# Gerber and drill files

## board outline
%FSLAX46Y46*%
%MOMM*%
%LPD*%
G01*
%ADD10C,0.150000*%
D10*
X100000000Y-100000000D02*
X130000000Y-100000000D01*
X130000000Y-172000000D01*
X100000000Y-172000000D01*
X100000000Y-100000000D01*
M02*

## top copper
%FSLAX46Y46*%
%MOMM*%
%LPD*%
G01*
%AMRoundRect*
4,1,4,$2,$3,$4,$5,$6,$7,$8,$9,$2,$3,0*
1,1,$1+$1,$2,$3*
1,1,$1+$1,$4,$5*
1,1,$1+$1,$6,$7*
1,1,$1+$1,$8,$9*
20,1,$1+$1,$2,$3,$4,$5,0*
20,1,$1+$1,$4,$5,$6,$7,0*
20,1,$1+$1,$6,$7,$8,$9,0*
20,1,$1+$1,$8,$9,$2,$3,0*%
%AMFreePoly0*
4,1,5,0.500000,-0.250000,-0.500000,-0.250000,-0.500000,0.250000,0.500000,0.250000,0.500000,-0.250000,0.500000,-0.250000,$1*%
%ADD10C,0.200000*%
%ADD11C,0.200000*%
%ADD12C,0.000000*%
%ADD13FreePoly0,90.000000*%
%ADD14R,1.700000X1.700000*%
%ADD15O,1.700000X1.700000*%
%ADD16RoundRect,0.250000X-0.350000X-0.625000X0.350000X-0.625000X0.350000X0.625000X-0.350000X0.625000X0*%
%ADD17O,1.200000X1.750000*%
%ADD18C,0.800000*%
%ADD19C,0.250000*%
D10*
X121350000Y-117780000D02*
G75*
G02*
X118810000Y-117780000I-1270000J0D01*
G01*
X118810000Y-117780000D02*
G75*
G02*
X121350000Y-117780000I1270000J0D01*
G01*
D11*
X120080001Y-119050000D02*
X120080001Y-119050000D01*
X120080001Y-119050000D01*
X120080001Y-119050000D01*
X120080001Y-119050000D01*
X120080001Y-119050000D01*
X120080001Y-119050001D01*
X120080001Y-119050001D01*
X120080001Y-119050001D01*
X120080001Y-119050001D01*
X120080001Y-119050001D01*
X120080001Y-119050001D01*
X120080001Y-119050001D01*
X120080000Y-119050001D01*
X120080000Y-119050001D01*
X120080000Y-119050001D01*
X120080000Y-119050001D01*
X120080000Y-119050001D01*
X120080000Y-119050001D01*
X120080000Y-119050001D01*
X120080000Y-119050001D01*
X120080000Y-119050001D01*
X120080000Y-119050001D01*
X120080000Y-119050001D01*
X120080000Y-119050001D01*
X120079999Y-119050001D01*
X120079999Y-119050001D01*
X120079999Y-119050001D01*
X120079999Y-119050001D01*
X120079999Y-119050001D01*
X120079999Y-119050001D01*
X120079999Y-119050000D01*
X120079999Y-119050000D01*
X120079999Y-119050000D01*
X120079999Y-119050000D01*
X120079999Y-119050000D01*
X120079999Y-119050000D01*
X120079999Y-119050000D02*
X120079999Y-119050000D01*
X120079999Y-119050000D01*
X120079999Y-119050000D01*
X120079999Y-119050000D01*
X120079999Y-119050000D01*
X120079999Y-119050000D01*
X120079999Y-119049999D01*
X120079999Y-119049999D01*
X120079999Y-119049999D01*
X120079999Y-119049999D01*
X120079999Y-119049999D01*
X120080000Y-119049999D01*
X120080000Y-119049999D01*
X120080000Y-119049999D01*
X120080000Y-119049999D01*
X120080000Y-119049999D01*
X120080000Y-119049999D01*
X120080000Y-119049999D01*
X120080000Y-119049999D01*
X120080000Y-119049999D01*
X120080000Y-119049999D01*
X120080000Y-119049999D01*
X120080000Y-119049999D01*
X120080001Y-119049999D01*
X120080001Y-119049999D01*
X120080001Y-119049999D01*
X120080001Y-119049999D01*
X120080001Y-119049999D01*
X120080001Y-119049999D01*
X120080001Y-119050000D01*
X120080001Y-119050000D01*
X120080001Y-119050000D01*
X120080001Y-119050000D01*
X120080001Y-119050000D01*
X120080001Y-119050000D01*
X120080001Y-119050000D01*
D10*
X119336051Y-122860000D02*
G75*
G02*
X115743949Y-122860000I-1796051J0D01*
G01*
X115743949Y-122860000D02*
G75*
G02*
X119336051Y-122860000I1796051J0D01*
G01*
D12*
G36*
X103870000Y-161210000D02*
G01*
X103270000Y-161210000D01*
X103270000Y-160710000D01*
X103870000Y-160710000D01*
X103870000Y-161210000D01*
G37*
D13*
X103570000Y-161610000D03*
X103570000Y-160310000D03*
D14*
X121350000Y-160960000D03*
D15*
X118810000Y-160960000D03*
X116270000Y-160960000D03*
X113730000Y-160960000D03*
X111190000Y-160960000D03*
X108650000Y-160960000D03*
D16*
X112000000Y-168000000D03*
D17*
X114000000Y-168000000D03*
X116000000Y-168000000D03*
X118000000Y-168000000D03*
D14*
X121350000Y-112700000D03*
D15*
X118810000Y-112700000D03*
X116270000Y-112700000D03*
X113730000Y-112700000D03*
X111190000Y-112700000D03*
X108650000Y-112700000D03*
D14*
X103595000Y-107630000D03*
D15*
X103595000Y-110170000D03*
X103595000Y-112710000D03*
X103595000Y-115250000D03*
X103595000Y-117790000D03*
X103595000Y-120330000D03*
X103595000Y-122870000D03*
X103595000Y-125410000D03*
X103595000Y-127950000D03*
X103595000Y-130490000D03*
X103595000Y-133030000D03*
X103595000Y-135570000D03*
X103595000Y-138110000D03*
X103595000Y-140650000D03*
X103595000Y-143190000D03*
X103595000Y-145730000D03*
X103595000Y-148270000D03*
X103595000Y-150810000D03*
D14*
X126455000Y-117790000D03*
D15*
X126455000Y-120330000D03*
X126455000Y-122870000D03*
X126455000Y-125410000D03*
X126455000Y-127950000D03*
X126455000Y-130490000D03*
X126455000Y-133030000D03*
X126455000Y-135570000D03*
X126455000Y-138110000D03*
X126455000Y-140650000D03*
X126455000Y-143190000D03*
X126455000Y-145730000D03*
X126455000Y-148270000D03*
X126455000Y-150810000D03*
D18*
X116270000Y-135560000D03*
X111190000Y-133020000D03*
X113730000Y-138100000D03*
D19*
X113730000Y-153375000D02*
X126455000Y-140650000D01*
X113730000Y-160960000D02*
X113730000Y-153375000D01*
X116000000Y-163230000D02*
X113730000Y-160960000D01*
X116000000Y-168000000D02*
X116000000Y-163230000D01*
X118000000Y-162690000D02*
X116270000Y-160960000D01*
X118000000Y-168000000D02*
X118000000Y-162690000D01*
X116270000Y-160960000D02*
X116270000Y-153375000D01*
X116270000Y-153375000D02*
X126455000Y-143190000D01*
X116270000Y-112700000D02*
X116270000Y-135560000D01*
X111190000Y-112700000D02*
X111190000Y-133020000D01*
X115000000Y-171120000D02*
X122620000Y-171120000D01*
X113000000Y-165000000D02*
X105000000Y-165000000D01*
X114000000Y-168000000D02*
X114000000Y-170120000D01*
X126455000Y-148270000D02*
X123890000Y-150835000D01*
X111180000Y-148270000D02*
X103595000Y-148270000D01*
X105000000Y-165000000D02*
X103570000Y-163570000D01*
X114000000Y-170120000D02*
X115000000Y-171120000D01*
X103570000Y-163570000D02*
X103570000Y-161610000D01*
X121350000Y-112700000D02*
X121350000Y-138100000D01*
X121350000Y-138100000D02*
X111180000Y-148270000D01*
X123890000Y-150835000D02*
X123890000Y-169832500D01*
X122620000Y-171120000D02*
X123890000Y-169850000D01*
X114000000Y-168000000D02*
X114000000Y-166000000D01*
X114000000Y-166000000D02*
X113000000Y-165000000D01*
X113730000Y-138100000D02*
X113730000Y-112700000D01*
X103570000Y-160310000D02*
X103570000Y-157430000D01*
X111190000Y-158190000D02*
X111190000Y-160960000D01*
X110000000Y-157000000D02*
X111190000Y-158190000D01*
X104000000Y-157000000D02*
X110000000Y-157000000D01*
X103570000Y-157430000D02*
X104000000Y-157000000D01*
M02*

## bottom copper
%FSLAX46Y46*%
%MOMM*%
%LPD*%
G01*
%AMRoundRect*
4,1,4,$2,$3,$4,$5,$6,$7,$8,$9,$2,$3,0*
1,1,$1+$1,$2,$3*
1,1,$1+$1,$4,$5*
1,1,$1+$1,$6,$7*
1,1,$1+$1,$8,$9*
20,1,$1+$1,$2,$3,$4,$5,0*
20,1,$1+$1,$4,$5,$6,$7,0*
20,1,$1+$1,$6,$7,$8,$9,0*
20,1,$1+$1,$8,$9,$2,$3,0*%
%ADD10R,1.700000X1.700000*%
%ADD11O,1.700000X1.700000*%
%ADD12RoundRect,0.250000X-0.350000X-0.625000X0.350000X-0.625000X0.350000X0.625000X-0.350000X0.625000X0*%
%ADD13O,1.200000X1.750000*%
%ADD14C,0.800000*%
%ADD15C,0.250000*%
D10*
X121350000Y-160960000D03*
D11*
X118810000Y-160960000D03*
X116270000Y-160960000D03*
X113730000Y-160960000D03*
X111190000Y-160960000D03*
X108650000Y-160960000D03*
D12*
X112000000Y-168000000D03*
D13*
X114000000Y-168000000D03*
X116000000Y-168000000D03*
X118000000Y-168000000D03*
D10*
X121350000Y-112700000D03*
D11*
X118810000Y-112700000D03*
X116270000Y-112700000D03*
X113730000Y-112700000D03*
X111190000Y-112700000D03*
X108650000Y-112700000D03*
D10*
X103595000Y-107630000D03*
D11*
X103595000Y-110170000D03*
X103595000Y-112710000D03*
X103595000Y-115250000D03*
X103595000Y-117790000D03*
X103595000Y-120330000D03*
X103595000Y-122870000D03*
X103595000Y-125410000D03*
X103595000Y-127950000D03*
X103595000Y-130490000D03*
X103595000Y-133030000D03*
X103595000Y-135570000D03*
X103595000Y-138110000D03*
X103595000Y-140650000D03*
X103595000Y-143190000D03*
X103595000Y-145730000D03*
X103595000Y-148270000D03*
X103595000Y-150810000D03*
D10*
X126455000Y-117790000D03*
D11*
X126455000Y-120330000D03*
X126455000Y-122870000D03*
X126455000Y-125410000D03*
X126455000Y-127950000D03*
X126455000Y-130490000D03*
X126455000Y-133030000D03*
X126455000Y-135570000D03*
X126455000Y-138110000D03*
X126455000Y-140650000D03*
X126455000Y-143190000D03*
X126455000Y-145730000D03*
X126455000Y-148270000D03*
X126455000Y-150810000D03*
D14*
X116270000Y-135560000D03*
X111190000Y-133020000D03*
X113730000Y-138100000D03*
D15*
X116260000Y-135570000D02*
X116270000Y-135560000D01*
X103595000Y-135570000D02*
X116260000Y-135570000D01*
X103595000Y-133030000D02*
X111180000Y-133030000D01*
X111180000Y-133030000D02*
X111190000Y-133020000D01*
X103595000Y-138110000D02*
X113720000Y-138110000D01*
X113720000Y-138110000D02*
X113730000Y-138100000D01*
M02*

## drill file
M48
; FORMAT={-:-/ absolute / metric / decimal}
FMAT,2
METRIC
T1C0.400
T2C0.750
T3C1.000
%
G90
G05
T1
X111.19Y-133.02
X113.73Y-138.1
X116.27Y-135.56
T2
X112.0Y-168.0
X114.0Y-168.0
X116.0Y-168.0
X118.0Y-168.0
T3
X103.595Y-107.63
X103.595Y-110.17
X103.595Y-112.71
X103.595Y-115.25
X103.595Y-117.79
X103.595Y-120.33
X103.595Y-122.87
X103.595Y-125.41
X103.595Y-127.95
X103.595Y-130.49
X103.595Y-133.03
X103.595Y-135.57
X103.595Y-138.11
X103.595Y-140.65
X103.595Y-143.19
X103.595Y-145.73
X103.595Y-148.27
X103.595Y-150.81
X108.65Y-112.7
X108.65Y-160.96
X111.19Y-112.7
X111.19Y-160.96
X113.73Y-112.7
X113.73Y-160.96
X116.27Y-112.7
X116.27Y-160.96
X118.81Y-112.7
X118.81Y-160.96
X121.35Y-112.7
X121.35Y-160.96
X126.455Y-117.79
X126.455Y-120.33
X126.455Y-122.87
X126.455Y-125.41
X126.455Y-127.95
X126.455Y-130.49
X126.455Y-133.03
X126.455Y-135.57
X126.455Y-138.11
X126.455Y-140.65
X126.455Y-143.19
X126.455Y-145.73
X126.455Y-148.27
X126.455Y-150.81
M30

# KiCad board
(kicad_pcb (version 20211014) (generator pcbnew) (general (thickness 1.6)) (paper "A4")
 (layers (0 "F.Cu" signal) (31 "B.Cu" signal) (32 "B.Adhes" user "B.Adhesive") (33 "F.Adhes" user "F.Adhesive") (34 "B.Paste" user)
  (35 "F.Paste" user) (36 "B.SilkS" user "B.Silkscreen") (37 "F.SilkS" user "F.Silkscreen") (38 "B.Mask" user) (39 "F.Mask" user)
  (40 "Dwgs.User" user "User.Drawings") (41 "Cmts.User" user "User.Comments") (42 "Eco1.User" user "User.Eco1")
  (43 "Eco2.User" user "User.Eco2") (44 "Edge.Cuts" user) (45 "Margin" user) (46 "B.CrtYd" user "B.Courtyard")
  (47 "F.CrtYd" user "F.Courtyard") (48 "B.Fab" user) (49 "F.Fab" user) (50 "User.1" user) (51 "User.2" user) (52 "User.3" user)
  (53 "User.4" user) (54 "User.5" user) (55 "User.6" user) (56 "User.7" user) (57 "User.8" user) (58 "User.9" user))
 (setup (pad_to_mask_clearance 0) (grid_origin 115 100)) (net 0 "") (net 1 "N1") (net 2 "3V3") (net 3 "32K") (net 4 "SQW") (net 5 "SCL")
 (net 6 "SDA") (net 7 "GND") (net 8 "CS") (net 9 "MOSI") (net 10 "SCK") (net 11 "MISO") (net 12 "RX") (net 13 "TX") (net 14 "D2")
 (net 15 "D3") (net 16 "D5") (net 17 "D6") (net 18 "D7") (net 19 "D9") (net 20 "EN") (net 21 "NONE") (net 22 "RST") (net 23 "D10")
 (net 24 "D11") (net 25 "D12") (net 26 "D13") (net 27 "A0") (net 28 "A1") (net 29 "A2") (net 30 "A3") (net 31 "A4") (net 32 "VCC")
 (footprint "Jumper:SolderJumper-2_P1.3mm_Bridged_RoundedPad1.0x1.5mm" (layer "F.Cu") (at 103.57 160.96 90)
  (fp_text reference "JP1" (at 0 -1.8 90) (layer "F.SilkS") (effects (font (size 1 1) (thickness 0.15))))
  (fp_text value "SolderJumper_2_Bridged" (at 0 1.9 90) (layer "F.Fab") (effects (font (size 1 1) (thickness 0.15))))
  (fp_poly (pts (xy 0.25 -0.3) (xy -0.25 -0.3) (xy -0.25 0.3) (xy 0.25 0.3)) (layer "F.Cu") (width 0) (fill solid))
  (pad "1" smd custom (at -0.65 0 90) (size 1 0.5) (layers "F.Cu" "F.Mask") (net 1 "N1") (zone_connect 2)
   (options (clearance outline) (anchor rect)) (primitives))
  (pad "2" smd custom (at 0.65 0 90) (size 1 0.5) (layers "F.Cu" "F.Mask") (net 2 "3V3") (zone_connect 2)
   (options (clearance outline) (anchor rect)) (primitives)))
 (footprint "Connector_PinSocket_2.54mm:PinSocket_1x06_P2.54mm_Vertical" (layer "F.Cu") (at 121.35 160.96 -90)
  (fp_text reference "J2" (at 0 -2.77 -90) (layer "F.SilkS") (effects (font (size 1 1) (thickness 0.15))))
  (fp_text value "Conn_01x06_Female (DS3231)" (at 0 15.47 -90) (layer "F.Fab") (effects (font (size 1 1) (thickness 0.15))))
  (pad "1" thru_hole rect (at 0 0 270) (size 1.7 1.7) (drill 1) (layers *.Cu *.Mask) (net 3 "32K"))
  (pad "2" thru_hole oval (at 0 2.54 270) (size 1.7 1.7) (drill 1) (layers *.Cu *.Mask) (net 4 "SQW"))
  (pad "3" thru_hole oval (at 0 5.08 270) (size 1.7 1.7) (drill 1) (layers *.Cu *.Mask) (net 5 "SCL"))
  (pad "4" thru_hole oval (at 0 7.62 270) (size 1.7 1.7) (drill 1) (layers *.Cu *.Mask) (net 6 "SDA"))
  (pad "5" thru_hole oval (at 0 10.16 270) (size 1.7 1.7) (drill 1) (layers *.Cu *.Mask) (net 1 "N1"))
  (pad "6" thru_hole oval (at 0 12.7 270) (size 1.7 1.7) (drill 1) (layers *.Cu *.Mask) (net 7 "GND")))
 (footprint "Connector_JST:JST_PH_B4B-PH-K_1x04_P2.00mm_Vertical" (layer "F.Cu") (at 112 168)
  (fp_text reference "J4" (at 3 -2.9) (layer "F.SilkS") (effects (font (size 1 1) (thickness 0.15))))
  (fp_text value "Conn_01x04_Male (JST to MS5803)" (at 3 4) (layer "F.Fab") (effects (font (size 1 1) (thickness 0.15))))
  (pad "1" thru_hole roundrect (at 0 0) (size 1.2 1.75) (drill 0.75) (layers *.Cu *.Mask) (roundrect_rratio 0.208333) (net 7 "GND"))
  (pad "2" thru_hole oval (at 2 0) (size 1.2 1.75) (drill 0.75) (layers *.Cu *.Mask) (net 2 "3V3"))
  (pad "3" thru_hole oval (at 4 0) (size 1.2 1.75) (drill 0.75) (layers *.Cu *.Mask) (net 6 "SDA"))
  (pad "4" thru_hole oval (at 6 0) (size 1.2 1.75) (drill 0.75) (layers *.Cu *.Mask) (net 5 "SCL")))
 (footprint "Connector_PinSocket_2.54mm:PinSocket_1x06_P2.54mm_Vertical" (layer "F.Cu") (at 121.35 112.7 -90)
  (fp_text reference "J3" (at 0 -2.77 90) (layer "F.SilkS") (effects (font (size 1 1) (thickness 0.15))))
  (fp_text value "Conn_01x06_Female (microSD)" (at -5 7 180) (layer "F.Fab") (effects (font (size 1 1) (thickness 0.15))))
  (pad "1" thru_hole rect (at 0 0 270) (size 1.7 1.7) (drill 1) (layers *.Cu *.Mask) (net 2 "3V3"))
  (pad "2" thru_hole oval (at 0 2.54 270) (size 1.7 1.7) (drill 1) (layers *.Cu *.Mask) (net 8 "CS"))
  (pad "3" thru_hole oval (at 0 5.08 270) (size 1.7 1.7) (drill 1) (layers *.Cu *.Mask) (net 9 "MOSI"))
  (pad "4" thru_hole oval (at 0 7.62 270) (size 1.7 1.7) (drill 1) (layers *.Cu *.Mask) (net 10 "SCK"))
  (pad "5" thru_hole oval (at 0 10.16 270) (size 1.7 1.7) (drill 1) (layers *.Cu *.Mask) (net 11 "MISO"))
  (pad "6" thru_hole oval (at 0 12.7 270) (size 1.7 1.7) (drill 1) (layers *.Cu *.Mask) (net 7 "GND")))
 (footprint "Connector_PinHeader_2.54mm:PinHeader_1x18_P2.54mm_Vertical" (layer "B.Cu") (at 103.595 107.63 180)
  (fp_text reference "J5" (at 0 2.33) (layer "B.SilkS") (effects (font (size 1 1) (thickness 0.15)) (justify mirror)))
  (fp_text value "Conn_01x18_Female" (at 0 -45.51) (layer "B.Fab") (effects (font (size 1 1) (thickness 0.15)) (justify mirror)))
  (pad "1" thru_hole rect (at 0 0 180) (size 1.7 1.7) (drill 1) (layers *.Cu *.Mask) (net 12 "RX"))
  (pad "2" thru_hole oval (at 0 -2.54 180) (size 1.7 1.7) (drill 1) (layers *.Cu *.Mask) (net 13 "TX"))
  (pad "3" thru_hole oval (at 0 -5.08 180) (size 1.7 1.7) (drill 1) (layers *.Cu *.Mask) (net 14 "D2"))
  (pad "4" thru_hole oval (at 0 -7.62 180) (size 1.7 1.7) (drill 1) (layers *.Cu *.Mask) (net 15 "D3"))
  (pad "5" thru_hole oval (at 0 -10.16 180) (size 1.7 1.7) (drill 1) (layers *.Cu *.Mask) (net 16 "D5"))
  (pad "6" thru_hole oval (at 0 -12.7 180) (size 1.7 1.7) (drill 1) (layers *.Cu *.Mask) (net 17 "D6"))
  (pad "7" thru_hole oval (at 0 -15.24 180) (size 1.7 1.7) (drill 1) (layers *.Cu *.Mask) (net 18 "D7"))
  (pad "8" thru_hole oval (at 0 -17.78 180) (size 1.7 1.7) (drill 1) (layers *.Cu *.Mask) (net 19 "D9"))
  (pad "9" thru_hole oval (at 0 -20.32 180) (size 1.7 1.7) (drill 1) (layers *.Cu *.Mask) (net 6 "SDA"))
  (pad "10" thru_hole oval (at 0 -22.86 180) (size 1.7 1.7) (drill 1) (layers *.Cu *.Mask) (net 5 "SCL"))
  (pad "11" thru_hole oval (at 0 -25.4 180) (size 1.7 1.7) (drill 1) (layers *.Cu *.Mask) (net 11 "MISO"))
  (pad "12" thru_hole oval (at 0 -27.94 180) (size 1.7 1.7) (drill 1) (layers *.Cu *.Mask) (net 9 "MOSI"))
  (pad "13" thru_hole oval (at 0 -30.48 180) (size 1.7 1.7) (drill 1) (layers *.Cu *.Mask) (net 10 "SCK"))
  (pad "14" thru_hole oval (at 0 -33.02 180) (size 1.7 1.7) (drill 1) (layers *.Cu *.Mask) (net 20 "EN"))
  (pad "15" thru_hole oval (at 0 -35.56 180) (size 1.7 1.7) (drill 1) (layers *.Cu *.Mask) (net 7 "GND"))
  (pad "16" thru_hole oval (at 0 -38.1 180) (size 1.7 1.7) (drill 1) (layers *.Cu *.Mask) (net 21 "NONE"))
  (pad "17" thru_hole oval (at 0 -40.64 180) (size 1.7 1.7) (drill 1) (layers *.Cu *.Mask) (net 2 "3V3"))
  (pad "18" thru_hole oval (at 0 -43.18 180) (size 1.7 1.7) (drill 1) (layers *.Cu *.Mask) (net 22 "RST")))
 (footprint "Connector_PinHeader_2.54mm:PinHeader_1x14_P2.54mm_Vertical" (layer "B.Cu") (at 126.455 117.79 180)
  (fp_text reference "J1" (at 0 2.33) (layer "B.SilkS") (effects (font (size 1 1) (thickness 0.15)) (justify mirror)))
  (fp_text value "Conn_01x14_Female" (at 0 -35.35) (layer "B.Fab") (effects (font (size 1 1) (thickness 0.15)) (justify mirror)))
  (pad "1" thru_hole rect (at 0 0 180) (size 1.7 1.7) (drill 1) (layers *.Cu *.Mask) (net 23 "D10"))
  (pad "2" thru_hole oval (at 0 -2.54 180) (size 1.7 1.7) (drill 1) (layers *.Cu *.Mask) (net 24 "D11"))
  (pad "3" thru_hole oval (at 0 -5.08 180) (size 1.7 1.7) (drill 1) (layers *.Cu *.Mask) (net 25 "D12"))
  (pad "4" thru_hole oval (at 0 -7.62 180) (size 1.7 1.7) (drill 1) (layers *.Cu *.Mask) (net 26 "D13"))
  (pad "5" thru_hole oval (at 0 -10.16 180) (size 1.7 1.7) (drill 1) (layers *.Cu *.Mask) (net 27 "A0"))
  (pad "6" thru_hole oval (at 0 -12.7 180) (size 1.7 1.7) (drill 1) (layers *.Cu *.Mask) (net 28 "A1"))
  (pad "7" thru_hole oval (at 0 -15.24 180) (size 1.7 1.7) (drill 1) (layers *.Cu *.Mask) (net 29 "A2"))
  (pad "8" thru_hole oval (at 0 -17.78 180) (size 1.7 1.7) (drill 1) (layers *.Cu *.Mask) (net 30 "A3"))
  (pad "9" thru_hole oval (at 0 -20.32 180) (size 1.7 1.7) (drill 1) (layers *.Cu *.Mask) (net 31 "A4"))
  (pad "10" thru_hole oval (at 0 -22.86 180) (size 1.7 1.7) (drill 1) (layers *.Cu *.Mask) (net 6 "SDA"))
  (pad "11" thru_hole oval (at 0 -25.4 180) (size 1.7 1.7) (drill 1) (layers *.Cu *.Mask) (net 5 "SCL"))
  (pad "12" thru_hole oval (at 0 -27.94 180) (size 1.7 1.7) (drill 1) (layers *.Cu *.Mask) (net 7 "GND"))
  (pad "13" thru_hole oval (at 0 -30.48 180) (size 1.7 1.7) (drill 1) (layers *.Cu *.Mask) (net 2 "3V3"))
  (pad "14" thru_hole oval (at 0 -33.02 180) (size 1.7 1.7) (drill 1) (layers *.Cu *.Mask) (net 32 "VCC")))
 (gr_circle (center 120.08 117.78) (end 118.81 117.78) (layer "F.Cu") (width 0.2) (fill none))
 (gr_circle (center 120.08 119.05) (end 120.08 119.05) (layer "F.Cu") (width 0.2) (fill none))
 (gr_circle (center 117.54 122.86) (end 118.81 121.59) (layer "F.Cu") (width 0.2) (fill none))
 (gr_rect (start 100 100) (end 130 172) (layer "Edge.Cuts") (width 0.15) (fill none))
 (segment (start 113.73 153.375) (end 126.455 140.65) (width 0.25) (layer "F.Cu") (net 6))
 (segment (start 113.73 160.96) (end 113.73 153.375) (width 0.25) (layer "F.Cu") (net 6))
 (segment (start 116 163.23) (end 113.73 160.96) (width 0.25) (layer "F.Cu") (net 6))
 (segment (start 116 168) (end 116 163.23) (width 0.25) (layer "F.Cu") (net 6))
 (segment (start 118 162.69) (end 116.27 160.96) (width 0.25) (layer "F.Cu") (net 5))
 (segment (start 118 168) (end 118 162.69) (width 0.25) (layer "F.Cu") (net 5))
 (segment (start 116.27 160.96) (end 116.27 153.375) (width 0.25) (layer "F.Cu") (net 5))
 (segment (start 116.27 153.375) (end 126.455 143.19) (width 0.25) (layer "F.Cu") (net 5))
 (segment (start 116.27 112.7) (end 116.27 135.56) (width 0.25) (layer "F.Cu") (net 9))
 (via (at 116.27 135.56) (size 0.8) (drill 0.4) (layers "F.Cu" "B.Cu") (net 9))
 (segment (start 116.26 135.57) (end 116.27 135.56) (width 0.25) (layer "B.Cu") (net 9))
 (segment (start 103.595 135.57) (end 116.26 135.57) (width 0.25) (layer "B.Cu") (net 9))
 (segment (start 111.19 112.7) (end 111.19 133.02) (width 0.25) (layer "F.Cu") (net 11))
 (via (at 111.19 133.02) (size 0.8) (drill 0.4) (layers "F.Cu" "B.Cu") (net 11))
 (segment (start 103.595 133.03) (end 111.18 133.03) (width 0.25) (layer "B.Cu") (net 11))
 (segment (start 111.18 133.03) (end 111.19 133.02) (width 0.25) (layer "B.Cu") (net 11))
 (segment (start 115 171.12) (end 122.62 171.12) (width 0.25) (layer "F.Cu") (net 2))
 (segment (start 113 165) (end 105 165) (width 0.25) (layer "F.Cu") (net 2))
 (segment (start 114 168) (end 114 170.12) (width 0.25) (layer "F.Cu") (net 2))
 (segment (start 126.455 148.27) (end 123.89 150.835) (width 0.25) (layer "F.Cu") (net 2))
 (segment (start 111.18 148.27) (end 103.595 148.27) (width 0.25) (layer "F.Cu") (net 2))
 (segment (start 105 165) (end 103.57 163.57) (width 0.25) (layer "F.Cu") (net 2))
 (segment (start 114 170.12) (end 115 171.12) (width 0.25) (layer "F.Cu") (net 2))
 (segment (start 103.57 163.57) (end 103.57 161.61) (width 0.25) (layer "F.Cu") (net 2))
 (segment (start 121.35 112.7) (end 121.35 138.1) (width 0.25) (layer "F.Cu") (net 2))
 (segment (start 121.35 138.1) (end 111.18 148.27) (width 0.25) (layer "F.Cu") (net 2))
 (segment (start 123.89 150.835) (end 123.89 169.8325) (width 0.25) (layer "F.Cu") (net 2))
 (segment (start 122.62 171.12) (end 123.89 169.85) (width 0.25) (layer "F.Cu") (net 2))
 (segment (start 114 168) (end 114 166) (width 0.25) (layer "F.Cu") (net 2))
 (segment (start 114 166) (end 113 165) (width 0.25) (layer "F.Cu") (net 2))
 (segment (start 113.73 138.1) (end 113.73 112.7) (width 0.25) (layer "F.Cu") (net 10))
 (via (at 113.73 138.1) (size 0.8) (drill 0.4) (layers "F.Cu" "B.Cu") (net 10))
 (segment (start 103.595 138.11) (end 113.72 138.11) (width 0.25) (layer "B.Cu") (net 10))
 (segment (start 113.72 138.11) (end 113.73 138.1) (width 0.25) (layer "B.Cu") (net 10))
 (segment (start 103.57 160.31) (end 103.57 157.43) (width 0.25) (layer "F.Cu") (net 1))
 (segment (start 111.19 158.19) (end 111.19 160.96) (width 0.25) (layer "F.Cu") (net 1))
 (segment (start 110 157) (end 111.19 158.19) (width 0.25) (layer "F.Cu") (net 1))
 (segment (start 104 157) (end 110 157) (width 0.25) (layer "F.Cu") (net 1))
 (segment (start 103.57 157.43) (end 104 157) (width 0.25) (layer "F.Cu") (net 1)))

